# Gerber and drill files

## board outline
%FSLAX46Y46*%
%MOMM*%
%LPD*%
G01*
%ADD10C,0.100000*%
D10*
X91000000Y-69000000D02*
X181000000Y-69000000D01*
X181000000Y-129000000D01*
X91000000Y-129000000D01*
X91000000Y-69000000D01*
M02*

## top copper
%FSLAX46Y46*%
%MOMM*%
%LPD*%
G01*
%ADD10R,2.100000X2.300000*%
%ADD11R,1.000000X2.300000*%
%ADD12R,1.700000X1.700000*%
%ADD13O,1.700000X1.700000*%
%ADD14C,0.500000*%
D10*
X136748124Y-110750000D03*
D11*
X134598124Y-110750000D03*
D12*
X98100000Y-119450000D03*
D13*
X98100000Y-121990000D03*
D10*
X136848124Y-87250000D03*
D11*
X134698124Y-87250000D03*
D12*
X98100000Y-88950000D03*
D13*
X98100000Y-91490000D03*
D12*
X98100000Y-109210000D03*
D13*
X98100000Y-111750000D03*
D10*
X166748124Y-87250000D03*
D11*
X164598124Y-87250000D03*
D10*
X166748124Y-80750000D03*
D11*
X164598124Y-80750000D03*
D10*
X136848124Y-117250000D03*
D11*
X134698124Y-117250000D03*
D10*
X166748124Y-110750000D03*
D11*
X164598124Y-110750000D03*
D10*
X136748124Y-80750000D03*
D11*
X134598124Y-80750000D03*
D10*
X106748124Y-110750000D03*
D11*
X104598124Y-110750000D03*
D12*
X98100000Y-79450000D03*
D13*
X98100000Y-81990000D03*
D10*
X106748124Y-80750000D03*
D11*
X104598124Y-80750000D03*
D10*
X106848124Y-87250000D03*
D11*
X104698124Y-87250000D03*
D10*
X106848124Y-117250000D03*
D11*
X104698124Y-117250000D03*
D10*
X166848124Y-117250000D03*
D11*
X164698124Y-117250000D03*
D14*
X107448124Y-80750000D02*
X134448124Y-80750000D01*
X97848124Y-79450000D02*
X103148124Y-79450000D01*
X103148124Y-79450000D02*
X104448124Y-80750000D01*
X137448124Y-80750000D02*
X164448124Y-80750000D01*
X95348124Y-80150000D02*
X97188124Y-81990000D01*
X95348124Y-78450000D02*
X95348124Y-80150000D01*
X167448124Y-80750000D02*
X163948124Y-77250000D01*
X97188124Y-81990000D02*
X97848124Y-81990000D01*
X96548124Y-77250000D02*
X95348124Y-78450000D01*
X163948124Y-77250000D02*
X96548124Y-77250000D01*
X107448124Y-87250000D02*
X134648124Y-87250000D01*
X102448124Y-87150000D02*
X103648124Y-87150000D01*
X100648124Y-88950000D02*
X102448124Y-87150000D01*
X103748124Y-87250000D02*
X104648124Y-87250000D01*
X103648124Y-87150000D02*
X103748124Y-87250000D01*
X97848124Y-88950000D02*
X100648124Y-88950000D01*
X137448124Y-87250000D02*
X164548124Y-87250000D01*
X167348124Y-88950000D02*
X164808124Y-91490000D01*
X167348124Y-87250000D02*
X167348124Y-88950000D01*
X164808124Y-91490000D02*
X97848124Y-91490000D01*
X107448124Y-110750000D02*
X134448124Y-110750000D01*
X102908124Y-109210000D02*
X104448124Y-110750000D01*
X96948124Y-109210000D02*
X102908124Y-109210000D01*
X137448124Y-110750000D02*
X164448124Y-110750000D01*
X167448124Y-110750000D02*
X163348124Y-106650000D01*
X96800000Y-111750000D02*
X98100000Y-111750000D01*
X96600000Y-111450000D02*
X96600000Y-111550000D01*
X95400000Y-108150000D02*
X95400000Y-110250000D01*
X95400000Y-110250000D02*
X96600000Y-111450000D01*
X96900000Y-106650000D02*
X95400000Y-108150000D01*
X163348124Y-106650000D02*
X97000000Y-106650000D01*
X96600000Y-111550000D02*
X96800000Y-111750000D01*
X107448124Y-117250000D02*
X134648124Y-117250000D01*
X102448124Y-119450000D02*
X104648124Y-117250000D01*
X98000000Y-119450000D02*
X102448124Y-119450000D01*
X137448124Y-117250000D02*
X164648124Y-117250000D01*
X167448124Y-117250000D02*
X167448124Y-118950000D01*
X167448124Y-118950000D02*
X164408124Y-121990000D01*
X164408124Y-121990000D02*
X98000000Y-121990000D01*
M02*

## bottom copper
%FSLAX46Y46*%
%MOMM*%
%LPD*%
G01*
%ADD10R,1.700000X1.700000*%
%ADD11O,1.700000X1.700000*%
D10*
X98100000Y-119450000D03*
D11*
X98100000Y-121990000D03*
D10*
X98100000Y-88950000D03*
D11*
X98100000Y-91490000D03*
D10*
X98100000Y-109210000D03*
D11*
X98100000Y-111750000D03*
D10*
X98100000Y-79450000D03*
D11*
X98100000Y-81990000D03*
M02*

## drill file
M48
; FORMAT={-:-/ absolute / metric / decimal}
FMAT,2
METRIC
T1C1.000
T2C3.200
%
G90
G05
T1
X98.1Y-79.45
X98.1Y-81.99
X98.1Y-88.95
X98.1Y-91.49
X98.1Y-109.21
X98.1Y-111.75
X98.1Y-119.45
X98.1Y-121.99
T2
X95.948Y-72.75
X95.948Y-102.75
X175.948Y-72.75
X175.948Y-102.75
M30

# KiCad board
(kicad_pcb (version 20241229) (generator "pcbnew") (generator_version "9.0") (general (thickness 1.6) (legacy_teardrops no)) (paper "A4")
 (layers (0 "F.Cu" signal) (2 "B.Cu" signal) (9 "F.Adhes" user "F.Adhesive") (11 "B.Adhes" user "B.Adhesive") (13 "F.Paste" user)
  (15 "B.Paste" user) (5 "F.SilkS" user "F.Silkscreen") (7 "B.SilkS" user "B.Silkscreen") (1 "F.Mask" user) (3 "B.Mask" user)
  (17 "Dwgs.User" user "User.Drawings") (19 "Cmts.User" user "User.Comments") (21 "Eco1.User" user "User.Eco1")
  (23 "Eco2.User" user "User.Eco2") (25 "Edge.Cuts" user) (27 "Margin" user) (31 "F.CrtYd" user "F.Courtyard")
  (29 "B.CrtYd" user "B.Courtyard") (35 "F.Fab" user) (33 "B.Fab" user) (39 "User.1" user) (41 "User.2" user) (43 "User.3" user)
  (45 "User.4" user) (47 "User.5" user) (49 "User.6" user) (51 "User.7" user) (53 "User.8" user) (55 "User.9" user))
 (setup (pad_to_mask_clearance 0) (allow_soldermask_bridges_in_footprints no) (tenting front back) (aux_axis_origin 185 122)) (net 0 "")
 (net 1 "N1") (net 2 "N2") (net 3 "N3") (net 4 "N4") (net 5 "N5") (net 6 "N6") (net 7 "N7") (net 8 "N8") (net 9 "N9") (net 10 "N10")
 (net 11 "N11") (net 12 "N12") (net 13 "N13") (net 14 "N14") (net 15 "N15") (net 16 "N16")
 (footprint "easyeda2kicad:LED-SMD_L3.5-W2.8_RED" (layer "F.Cu") (at 135.948124 110.75)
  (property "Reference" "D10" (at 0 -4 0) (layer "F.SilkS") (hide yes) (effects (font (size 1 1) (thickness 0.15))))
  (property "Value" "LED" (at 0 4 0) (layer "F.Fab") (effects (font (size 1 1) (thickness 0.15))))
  (pad "1" smd rect (at 0.8 0) (size 2.1 2.3) (layers "F.Cu" "F.Mask" "F.Paste") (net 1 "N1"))
  (pad "2" smd rect (at -1.35 0) (size 1 2.3) (layers "F.Cu" "F.Mask" "F.Paste") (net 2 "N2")))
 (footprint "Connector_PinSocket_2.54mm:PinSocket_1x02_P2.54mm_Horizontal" (layer "F.Cu") (at 98.1 119.45)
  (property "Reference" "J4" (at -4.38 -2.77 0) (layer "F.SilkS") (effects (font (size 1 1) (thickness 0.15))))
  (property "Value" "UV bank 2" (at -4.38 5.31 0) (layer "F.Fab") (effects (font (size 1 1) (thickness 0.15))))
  (pad "1" thru_hole rect (at 0 0) (size 1.7 1.7) (drill 1) (layers "*.Cu" "*.Mask") (remove_unused_layers no) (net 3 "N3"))
  (pad "2" thru_hole oval (at 0 2.54) (size 1.7 1.7) (drill 1) (layers "*.Cu" "*.Mask") (remove_unused_layers no) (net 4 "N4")))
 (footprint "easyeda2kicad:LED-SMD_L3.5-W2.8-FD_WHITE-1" (layer "F.Cu") (at 136.048124 87.25)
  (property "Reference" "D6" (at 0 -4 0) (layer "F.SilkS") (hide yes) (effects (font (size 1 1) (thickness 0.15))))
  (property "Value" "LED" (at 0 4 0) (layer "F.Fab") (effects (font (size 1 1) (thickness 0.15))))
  (pad "1" smd rect (at 0.8 0 180) (size 2.1 2.3) (layers "F.Cu" "F.Mask" "F.Paste") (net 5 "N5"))
  (pad "2" smd rect (at -1.35 0 180) (size 1 2.3) (layers "F.Cu" "F.Mask" "F.Paste") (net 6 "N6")))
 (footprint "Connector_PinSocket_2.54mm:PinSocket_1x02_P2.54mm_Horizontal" (layer "F.Cu") (at 98.1 88.95)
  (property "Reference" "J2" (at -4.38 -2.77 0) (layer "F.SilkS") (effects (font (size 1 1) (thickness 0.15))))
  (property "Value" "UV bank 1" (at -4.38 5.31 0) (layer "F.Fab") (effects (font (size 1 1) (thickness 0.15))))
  (pad "1" thru_hole rect (at 0 0) (size 1.7 1.7) (drill 1) (layers "*.Cu" "*.Mask") (remove_unused_layers no) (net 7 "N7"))
  (pad "2" thru_hole oval (at 0 2.54) (size 1.7 1.7) (drill 1) (layers "*.Cu" "*.Mask") (remove_unused_layers no) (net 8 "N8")))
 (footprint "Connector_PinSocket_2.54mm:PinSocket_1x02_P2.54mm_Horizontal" (layer "F.Cu") (at 98.1 109.21)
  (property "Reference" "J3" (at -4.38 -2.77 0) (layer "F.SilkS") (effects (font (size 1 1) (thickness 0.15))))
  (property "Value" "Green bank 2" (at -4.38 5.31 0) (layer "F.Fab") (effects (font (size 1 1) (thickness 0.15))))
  (pad "1" thru_hole rect (at 0 0) (size 1.7 1.7) (drill 1) (layers "*.Cu" "*.Mask") (remove_unused_layers no) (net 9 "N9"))
  (pad "2" thru_hole oval (at 0 2.54) (size 1.7 1.7) (drill 1) (layers "*.Cu" "*.Mask") (remove_unused_layers no) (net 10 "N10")))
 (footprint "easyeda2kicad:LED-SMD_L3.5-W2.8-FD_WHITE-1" (layer "F.Cu") (at 165.948124 87.25)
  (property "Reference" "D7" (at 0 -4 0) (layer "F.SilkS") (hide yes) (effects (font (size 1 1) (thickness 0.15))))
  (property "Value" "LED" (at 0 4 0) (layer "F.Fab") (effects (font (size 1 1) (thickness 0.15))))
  (pad "1" smd rect (at 0.8 0 180) (size 2.1 2.3) (layers "F.Cu" "F.Mask" "F.Paste") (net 8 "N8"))
  (pad "2" smd rect (at -1.35 0 180) (size 1 2.3) (layers "F.Cu" "F.Mask" "F.Paste") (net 5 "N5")))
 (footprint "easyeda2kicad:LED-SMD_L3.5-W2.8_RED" (layer "F.Cu") (at 165.948124 80.75)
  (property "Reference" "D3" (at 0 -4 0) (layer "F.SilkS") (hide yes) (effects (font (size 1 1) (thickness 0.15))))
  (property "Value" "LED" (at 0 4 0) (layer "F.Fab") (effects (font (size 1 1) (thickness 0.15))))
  (pad "1" smd rect (at 0.8 0) (size 2.1 2.3) (layers "F.Cu" "F.Mask" "F.Paste") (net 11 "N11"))
  (pad "2" smd rect (at -1.35 0) (size 1 2.3) (layers "F.Cu" "F.Mask" "F.Paste") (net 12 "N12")))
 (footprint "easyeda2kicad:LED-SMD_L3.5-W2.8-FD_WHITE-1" (layer "F.Cu") (at 136.048124 117.25)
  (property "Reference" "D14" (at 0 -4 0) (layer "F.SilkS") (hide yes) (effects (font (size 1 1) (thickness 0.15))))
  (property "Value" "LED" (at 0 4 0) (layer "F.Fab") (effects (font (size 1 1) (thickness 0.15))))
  (pad "1" smd rect (at 0.8 0 180) (size 2.1 2.3) (layers "F.Cu" "F.Mask" "F.Paste") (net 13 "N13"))
  (pad "2" smd rect (at -1.35 0 180) (size 1 2.3) (layers "F.Cu" "F.Mask" "F.Paste") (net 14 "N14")))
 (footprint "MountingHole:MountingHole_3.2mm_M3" (layer "F.Cu") (at 175.948124 72.75)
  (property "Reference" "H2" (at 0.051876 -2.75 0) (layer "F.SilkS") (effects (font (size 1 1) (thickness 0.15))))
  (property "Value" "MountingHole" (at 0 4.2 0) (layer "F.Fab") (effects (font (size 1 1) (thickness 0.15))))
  (pad "" np_thru_hole circle (at 0 0) (size 3.2 3.2) (drill 3.2) (layers "*.Cu" "*.Mask")))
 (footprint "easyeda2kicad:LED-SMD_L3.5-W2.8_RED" (layer "F.Cu") (at 165.948124 110.75)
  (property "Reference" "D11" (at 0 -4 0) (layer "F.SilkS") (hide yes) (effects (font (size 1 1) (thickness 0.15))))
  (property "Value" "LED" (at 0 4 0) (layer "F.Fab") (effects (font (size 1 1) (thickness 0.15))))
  (pad "1" smd rect (at 0.8 0) (size 2.1 2.3) (layers "F.Cu" "F.Mask" "F.Paste") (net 10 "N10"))
  (pad "2" smd rect (at -1.35 0) (size 1 2.3) (layers "F.Cu" "F.Mask" "F.Paste") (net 1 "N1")))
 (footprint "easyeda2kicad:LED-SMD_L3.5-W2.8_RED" (layer "F.Cu") (at 135.948124 80.75)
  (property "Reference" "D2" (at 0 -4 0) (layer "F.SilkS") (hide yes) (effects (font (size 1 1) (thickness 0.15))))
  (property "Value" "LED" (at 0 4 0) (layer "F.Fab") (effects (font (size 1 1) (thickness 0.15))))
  (pad "1" smd rect (at 0.8 0) (size 2.1 2.3) (layers "F.Cu" "F.Mask" "F.Paste") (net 12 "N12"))
  (pad "2" smd rect (at -1.35 0) (size 1 2.3) (layers "F.Cu" "F.Mask" "F.Paste") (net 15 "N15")))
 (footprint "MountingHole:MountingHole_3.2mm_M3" (layer "F.Cu") (at 95.948124 102.75)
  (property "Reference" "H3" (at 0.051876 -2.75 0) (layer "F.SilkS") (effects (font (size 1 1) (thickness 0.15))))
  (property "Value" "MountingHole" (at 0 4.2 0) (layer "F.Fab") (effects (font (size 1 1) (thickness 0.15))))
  (pad "" np_thru_hole circle (at 0 0) (size 3.2 3.2) (drill 3.2) (layers "*.Cu" "*.Mask")))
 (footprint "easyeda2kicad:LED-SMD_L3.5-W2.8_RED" (layer "F.Cu") (at 105.948124 110.75)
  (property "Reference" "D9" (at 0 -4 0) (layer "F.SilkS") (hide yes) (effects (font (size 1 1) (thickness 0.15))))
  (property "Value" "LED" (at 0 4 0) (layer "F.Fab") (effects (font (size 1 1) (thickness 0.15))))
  (pad "1" smd rect (at 0.8 0) (size 2.1 2.3) (layers "F.Cu" "F.Mask" "F.Paste") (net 2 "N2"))
  (pad "2" smd rect (at -1.35 0) (size 1 2.3) (layers "F.Cu" "F.Mask" "F.Paste") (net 9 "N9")))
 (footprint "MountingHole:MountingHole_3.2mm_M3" (layer "F.Cu") (at 175.948124 102.75)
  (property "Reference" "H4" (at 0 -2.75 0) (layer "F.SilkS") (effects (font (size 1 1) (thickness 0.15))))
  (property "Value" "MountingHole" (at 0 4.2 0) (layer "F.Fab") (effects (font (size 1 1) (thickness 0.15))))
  (pad "" np_thru_hole circle (at 0 0) (size 3.2 3.2) (drill 3.2) (layers "*.Cu" "*.Mask")))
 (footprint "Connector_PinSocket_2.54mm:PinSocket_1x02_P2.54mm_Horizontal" (layer "F.Cu") (at 98.1 79.45)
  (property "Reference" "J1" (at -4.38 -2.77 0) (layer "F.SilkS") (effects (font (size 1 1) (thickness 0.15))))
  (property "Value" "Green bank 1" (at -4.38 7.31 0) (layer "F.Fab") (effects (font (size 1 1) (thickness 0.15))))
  (pad "1" thru_hole rect (at 0 0) (size 1.7 1.7) (drill 1) (layers "*.Cu" "*.Mask") (remove_unused_layers no) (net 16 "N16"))
  (pad "2" thru_hole oval (at 0 2.54) (size 1.7 1.7) (drill 1) (layers "*.Cu" "*.Mask") (remove_unused_layers no) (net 11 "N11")))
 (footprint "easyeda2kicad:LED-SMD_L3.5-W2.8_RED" (layer "F.Cu") (at 105.948124 80.75)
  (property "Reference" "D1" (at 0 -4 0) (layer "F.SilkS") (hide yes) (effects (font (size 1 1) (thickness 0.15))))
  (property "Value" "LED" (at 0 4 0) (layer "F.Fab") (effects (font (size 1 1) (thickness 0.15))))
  (pad "1" smd rect (at 0.8 0) (size 2.1 2.3) (layers "F.Cu" "F.Mask" "F.Paste") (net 15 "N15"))
  (pad "2" smd rect (at -1.35 0) (size 1 2.3) (layers "F.Cu" "F.Mask" "F.Paste") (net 16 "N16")))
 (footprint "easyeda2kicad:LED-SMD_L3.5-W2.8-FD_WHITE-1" (layer "F.Cu") (at 106.048124 87.25)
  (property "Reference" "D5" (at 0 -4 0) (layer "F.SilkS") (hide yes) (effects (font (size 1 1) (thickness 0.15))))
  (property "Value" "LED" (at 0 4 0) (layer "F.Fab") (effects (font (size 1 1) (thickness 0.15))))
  (pad "1" smd rect (at 0.8 0 180) (size 2.1 2.3) (layers "F.Cu" "F.Mask" "F.Paste") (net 6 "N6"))
  (pad "2" smd rect (at -1.35 0 180) (size 1 2.3) (layers "F.Cu" "F.Mask" "F.Paste") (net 7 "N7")))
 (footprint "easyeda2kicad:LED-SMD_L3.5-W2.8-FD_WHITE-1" (layer "F.Cu") (at 106.048124 117.25)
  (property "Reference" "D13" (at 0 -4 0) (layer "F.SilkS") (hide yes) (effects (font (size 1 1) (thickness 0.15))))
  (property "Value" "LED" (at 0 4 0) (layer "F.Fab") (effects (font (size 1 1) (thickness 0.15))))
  (pad "1" smd rect (at 0.8 0 180) (size 2.1 2.3) (layers "F.Cu" "F.Mask" "F.Paste") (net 14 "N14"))
  (pad "2" smd rect (at -1.35 0 180) (size 1 2.3) (layers "F.Cu" "F.Mask" "F.Paste") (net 3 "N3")))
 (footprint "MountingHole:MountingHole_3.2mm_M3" (layer "F.Cu") (at 95.948124 72.75)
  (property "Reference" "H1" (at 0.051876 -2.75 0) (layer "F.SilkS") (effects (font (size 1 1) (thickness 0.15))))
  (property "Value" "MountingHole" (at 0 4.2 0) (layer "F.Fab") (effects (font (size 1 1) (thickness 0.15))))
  (pad "" np_thru_hole circle (at 0 0) (size 3.2 3.2) (drill 3.2) (layers "*.Cu" "*.Mask")))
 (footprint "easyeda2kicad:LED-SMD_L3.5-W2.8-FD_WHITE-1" (layer "F.Cu") (at 166.048124 117.25)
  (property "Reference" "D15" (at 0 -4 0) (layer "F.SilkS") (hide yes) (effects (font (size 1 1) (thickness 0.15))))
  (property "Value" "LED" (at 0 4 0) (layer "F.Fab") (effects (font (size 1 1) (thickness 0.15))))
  (pad "1" smd rect (at 0.8 0 180) (size 2.1 2.3) (layers "F.Cu" "F.Mask" "F.Paste") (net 4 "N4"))
  (pad "2" smd rect (at -1.35 0 180) (size 1 2.3) (layers "F.Cu" "F.Mask" "F.Paste") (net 13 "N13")))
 (gr_rect (start 91 69) (end 181 129) (stroke (width 0.1) (type solid)) (fill no) (layer "Edge.Cuts"))
 (segment (start 107.448124 80.75) (end 134.448124 80.75) (width 0.5) (layer "F.Cu") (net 15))
 (segment (start 97.848124 79.45) (end 103.148124 79.45) (width 0.5) (layer "F.Cu") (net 16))
 (segment (start 103.148124 79.45) (end 104.448124 80.75) (width 0.5) (layer "F.Cu") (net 16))
 (segment (start 137.448124 80.75) (end 164.448124 80.75) (width 0.5) (layer "F.Cu") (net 12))
 (segment (start 95.348124 80.15) (end 97.188124 81.99) (width 0.5) (layer "F.Cu") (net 11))
 (segment (start 95.348124 78.45) (end 95.348124 80.15) (width 0.5) (layer "F.Cu") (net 11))
 (segment (start 167.448124 80.75) (end 163.948124 77.25) (width 0.5) (layer "F.Cu") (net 11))
 (segment (start 97.188124 81.99) (end 97.848124 81.99) (width 0.5) (layer "F.Cu") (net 11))
 (segment (start 96.548124 77.25) (end 95.348124 78.45) (width 0.5) (layer "F.Cu") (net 11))
 (segment (start 163.948124 77.25) (end 96.548124 77.25) (width 0.5) (layer "F.Cu") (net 11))
 (segment (start 107.448124 87.25) (end 134.648124 87.25) (width 0.5) (layer "F.Cu") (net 6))
 (segment (start 102.448124 87.15) (end 103.648124 87.15) (width 0.5) (layer "F.Cu") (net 7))
 (segment (start 100.648124 88.95) (end 102.448124 87.15) (width 0.5) (layer "F.Cu") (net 7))
 (segment (start 103.748124 87.25) (end 104.648124 87.25) (width 0.5) (layer "F.Cu") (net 7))
 (segment (start 103.648124 87.15) (end 103.748124 87.25) (width 0.5) (layer "F.Cu") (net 7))
 (segment (start 97.848124 88.95) (end 100.648124 88.95) (width 0.5) (layer "F.Cu") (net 7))
 (segment (start 137.448124 87.25) (end 164.548124 87.25) (width 0.5) (layer "F.Cu") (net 5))
 (segment (start 167.348124 88.95) (end 164.808124 91.49) (width 0.5) (layer "F.Cu") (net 8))
 (segment (start 167.348124 87.25) (end 167.348124 88.95) (width 0.5) (layer "F.Cu") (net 8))
 (segment (start 164.808124 91.49) (end 97.848124 91.49) (width 0.5) (layer "F.Cu") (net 8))
 (segment (start 107.448124 110.75) (end 134.448124 110.75) (width 0.5) (layer "F.Cu") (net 2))
 (segment (start 102.908124 109.21) (end 104.448124 110.75) (width 0.5) (layer "F.Cu") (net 9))
 (segment (start 96.948124 109.21) (end 102.908124 109.21) (width 0.5) (layer "F.Cu") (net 9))
 (segment (start 137.448124 110.75) (end 164.448124 110.75) (width 0.5) (layer "F.Cu") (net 1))
 (segment (start 167.448124 110.75) (end 163.348124 106.65) (width 0.5) (layer "F.Cu") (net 10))
 (segment (start 96.8 111.75) (end 98.1 111.75) (width 0.5) (layer "F.Cu") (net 10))
 (segment (start 96.6 111.45) (end 96.6 111.55) (width 0.5) (layer "F.Cu") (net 10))
 (segment (start 95.4 108.15) (end 95.4 110.25) (width 0.5) (layer "F.Cu") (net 10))
 (segment (start 95.4 110.25) (end 96.6 111.45) (width 0.5) (layer "F.Cu") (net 10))
 (segment (start 96.9 106.65) (end 95.4 108.15) (width 0.5) (layer "F.Cu") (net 10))
 (segment (start 163.348124 106.65) (end 97 106.65) (width 0.5) (layer "F.Cu") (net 10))
 (segment (start 96.6 111.55) (end 96.8 111.75) (width 0.5) (layer "F.Cu") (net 10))
 (segment (start 107.448124 117.25) (end 134.648124 117.25) (width 0.5) (layer "F.Cu") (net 14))
 (segment (start 102.448124 119.45) (end 104.648124 117.25) (width 0.5) (layer "F.Cu") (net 3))
 (segment (start 98 119.45) (end 102.448124 119.45) (width 0.5) (layer "F.Cu") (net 3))
 (segment (start 137.448124 117.25) (end 164.648124 117.25) (width 0.5) (layer "F.Cu") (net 13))
 (segment (start 167.448124 117.25) (end 167.448124 118.95) (width 0.5) (layer "F.Cu") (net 4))
 (segment (start 167.448124 118.95) (end 164.408124 121.99) (width 0.5) (layer "F.Cu") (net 4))
 (segment (start 164.408124 121.99) (end 98 121.99) (width 0.5) (layer "F.Cu") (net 4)))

